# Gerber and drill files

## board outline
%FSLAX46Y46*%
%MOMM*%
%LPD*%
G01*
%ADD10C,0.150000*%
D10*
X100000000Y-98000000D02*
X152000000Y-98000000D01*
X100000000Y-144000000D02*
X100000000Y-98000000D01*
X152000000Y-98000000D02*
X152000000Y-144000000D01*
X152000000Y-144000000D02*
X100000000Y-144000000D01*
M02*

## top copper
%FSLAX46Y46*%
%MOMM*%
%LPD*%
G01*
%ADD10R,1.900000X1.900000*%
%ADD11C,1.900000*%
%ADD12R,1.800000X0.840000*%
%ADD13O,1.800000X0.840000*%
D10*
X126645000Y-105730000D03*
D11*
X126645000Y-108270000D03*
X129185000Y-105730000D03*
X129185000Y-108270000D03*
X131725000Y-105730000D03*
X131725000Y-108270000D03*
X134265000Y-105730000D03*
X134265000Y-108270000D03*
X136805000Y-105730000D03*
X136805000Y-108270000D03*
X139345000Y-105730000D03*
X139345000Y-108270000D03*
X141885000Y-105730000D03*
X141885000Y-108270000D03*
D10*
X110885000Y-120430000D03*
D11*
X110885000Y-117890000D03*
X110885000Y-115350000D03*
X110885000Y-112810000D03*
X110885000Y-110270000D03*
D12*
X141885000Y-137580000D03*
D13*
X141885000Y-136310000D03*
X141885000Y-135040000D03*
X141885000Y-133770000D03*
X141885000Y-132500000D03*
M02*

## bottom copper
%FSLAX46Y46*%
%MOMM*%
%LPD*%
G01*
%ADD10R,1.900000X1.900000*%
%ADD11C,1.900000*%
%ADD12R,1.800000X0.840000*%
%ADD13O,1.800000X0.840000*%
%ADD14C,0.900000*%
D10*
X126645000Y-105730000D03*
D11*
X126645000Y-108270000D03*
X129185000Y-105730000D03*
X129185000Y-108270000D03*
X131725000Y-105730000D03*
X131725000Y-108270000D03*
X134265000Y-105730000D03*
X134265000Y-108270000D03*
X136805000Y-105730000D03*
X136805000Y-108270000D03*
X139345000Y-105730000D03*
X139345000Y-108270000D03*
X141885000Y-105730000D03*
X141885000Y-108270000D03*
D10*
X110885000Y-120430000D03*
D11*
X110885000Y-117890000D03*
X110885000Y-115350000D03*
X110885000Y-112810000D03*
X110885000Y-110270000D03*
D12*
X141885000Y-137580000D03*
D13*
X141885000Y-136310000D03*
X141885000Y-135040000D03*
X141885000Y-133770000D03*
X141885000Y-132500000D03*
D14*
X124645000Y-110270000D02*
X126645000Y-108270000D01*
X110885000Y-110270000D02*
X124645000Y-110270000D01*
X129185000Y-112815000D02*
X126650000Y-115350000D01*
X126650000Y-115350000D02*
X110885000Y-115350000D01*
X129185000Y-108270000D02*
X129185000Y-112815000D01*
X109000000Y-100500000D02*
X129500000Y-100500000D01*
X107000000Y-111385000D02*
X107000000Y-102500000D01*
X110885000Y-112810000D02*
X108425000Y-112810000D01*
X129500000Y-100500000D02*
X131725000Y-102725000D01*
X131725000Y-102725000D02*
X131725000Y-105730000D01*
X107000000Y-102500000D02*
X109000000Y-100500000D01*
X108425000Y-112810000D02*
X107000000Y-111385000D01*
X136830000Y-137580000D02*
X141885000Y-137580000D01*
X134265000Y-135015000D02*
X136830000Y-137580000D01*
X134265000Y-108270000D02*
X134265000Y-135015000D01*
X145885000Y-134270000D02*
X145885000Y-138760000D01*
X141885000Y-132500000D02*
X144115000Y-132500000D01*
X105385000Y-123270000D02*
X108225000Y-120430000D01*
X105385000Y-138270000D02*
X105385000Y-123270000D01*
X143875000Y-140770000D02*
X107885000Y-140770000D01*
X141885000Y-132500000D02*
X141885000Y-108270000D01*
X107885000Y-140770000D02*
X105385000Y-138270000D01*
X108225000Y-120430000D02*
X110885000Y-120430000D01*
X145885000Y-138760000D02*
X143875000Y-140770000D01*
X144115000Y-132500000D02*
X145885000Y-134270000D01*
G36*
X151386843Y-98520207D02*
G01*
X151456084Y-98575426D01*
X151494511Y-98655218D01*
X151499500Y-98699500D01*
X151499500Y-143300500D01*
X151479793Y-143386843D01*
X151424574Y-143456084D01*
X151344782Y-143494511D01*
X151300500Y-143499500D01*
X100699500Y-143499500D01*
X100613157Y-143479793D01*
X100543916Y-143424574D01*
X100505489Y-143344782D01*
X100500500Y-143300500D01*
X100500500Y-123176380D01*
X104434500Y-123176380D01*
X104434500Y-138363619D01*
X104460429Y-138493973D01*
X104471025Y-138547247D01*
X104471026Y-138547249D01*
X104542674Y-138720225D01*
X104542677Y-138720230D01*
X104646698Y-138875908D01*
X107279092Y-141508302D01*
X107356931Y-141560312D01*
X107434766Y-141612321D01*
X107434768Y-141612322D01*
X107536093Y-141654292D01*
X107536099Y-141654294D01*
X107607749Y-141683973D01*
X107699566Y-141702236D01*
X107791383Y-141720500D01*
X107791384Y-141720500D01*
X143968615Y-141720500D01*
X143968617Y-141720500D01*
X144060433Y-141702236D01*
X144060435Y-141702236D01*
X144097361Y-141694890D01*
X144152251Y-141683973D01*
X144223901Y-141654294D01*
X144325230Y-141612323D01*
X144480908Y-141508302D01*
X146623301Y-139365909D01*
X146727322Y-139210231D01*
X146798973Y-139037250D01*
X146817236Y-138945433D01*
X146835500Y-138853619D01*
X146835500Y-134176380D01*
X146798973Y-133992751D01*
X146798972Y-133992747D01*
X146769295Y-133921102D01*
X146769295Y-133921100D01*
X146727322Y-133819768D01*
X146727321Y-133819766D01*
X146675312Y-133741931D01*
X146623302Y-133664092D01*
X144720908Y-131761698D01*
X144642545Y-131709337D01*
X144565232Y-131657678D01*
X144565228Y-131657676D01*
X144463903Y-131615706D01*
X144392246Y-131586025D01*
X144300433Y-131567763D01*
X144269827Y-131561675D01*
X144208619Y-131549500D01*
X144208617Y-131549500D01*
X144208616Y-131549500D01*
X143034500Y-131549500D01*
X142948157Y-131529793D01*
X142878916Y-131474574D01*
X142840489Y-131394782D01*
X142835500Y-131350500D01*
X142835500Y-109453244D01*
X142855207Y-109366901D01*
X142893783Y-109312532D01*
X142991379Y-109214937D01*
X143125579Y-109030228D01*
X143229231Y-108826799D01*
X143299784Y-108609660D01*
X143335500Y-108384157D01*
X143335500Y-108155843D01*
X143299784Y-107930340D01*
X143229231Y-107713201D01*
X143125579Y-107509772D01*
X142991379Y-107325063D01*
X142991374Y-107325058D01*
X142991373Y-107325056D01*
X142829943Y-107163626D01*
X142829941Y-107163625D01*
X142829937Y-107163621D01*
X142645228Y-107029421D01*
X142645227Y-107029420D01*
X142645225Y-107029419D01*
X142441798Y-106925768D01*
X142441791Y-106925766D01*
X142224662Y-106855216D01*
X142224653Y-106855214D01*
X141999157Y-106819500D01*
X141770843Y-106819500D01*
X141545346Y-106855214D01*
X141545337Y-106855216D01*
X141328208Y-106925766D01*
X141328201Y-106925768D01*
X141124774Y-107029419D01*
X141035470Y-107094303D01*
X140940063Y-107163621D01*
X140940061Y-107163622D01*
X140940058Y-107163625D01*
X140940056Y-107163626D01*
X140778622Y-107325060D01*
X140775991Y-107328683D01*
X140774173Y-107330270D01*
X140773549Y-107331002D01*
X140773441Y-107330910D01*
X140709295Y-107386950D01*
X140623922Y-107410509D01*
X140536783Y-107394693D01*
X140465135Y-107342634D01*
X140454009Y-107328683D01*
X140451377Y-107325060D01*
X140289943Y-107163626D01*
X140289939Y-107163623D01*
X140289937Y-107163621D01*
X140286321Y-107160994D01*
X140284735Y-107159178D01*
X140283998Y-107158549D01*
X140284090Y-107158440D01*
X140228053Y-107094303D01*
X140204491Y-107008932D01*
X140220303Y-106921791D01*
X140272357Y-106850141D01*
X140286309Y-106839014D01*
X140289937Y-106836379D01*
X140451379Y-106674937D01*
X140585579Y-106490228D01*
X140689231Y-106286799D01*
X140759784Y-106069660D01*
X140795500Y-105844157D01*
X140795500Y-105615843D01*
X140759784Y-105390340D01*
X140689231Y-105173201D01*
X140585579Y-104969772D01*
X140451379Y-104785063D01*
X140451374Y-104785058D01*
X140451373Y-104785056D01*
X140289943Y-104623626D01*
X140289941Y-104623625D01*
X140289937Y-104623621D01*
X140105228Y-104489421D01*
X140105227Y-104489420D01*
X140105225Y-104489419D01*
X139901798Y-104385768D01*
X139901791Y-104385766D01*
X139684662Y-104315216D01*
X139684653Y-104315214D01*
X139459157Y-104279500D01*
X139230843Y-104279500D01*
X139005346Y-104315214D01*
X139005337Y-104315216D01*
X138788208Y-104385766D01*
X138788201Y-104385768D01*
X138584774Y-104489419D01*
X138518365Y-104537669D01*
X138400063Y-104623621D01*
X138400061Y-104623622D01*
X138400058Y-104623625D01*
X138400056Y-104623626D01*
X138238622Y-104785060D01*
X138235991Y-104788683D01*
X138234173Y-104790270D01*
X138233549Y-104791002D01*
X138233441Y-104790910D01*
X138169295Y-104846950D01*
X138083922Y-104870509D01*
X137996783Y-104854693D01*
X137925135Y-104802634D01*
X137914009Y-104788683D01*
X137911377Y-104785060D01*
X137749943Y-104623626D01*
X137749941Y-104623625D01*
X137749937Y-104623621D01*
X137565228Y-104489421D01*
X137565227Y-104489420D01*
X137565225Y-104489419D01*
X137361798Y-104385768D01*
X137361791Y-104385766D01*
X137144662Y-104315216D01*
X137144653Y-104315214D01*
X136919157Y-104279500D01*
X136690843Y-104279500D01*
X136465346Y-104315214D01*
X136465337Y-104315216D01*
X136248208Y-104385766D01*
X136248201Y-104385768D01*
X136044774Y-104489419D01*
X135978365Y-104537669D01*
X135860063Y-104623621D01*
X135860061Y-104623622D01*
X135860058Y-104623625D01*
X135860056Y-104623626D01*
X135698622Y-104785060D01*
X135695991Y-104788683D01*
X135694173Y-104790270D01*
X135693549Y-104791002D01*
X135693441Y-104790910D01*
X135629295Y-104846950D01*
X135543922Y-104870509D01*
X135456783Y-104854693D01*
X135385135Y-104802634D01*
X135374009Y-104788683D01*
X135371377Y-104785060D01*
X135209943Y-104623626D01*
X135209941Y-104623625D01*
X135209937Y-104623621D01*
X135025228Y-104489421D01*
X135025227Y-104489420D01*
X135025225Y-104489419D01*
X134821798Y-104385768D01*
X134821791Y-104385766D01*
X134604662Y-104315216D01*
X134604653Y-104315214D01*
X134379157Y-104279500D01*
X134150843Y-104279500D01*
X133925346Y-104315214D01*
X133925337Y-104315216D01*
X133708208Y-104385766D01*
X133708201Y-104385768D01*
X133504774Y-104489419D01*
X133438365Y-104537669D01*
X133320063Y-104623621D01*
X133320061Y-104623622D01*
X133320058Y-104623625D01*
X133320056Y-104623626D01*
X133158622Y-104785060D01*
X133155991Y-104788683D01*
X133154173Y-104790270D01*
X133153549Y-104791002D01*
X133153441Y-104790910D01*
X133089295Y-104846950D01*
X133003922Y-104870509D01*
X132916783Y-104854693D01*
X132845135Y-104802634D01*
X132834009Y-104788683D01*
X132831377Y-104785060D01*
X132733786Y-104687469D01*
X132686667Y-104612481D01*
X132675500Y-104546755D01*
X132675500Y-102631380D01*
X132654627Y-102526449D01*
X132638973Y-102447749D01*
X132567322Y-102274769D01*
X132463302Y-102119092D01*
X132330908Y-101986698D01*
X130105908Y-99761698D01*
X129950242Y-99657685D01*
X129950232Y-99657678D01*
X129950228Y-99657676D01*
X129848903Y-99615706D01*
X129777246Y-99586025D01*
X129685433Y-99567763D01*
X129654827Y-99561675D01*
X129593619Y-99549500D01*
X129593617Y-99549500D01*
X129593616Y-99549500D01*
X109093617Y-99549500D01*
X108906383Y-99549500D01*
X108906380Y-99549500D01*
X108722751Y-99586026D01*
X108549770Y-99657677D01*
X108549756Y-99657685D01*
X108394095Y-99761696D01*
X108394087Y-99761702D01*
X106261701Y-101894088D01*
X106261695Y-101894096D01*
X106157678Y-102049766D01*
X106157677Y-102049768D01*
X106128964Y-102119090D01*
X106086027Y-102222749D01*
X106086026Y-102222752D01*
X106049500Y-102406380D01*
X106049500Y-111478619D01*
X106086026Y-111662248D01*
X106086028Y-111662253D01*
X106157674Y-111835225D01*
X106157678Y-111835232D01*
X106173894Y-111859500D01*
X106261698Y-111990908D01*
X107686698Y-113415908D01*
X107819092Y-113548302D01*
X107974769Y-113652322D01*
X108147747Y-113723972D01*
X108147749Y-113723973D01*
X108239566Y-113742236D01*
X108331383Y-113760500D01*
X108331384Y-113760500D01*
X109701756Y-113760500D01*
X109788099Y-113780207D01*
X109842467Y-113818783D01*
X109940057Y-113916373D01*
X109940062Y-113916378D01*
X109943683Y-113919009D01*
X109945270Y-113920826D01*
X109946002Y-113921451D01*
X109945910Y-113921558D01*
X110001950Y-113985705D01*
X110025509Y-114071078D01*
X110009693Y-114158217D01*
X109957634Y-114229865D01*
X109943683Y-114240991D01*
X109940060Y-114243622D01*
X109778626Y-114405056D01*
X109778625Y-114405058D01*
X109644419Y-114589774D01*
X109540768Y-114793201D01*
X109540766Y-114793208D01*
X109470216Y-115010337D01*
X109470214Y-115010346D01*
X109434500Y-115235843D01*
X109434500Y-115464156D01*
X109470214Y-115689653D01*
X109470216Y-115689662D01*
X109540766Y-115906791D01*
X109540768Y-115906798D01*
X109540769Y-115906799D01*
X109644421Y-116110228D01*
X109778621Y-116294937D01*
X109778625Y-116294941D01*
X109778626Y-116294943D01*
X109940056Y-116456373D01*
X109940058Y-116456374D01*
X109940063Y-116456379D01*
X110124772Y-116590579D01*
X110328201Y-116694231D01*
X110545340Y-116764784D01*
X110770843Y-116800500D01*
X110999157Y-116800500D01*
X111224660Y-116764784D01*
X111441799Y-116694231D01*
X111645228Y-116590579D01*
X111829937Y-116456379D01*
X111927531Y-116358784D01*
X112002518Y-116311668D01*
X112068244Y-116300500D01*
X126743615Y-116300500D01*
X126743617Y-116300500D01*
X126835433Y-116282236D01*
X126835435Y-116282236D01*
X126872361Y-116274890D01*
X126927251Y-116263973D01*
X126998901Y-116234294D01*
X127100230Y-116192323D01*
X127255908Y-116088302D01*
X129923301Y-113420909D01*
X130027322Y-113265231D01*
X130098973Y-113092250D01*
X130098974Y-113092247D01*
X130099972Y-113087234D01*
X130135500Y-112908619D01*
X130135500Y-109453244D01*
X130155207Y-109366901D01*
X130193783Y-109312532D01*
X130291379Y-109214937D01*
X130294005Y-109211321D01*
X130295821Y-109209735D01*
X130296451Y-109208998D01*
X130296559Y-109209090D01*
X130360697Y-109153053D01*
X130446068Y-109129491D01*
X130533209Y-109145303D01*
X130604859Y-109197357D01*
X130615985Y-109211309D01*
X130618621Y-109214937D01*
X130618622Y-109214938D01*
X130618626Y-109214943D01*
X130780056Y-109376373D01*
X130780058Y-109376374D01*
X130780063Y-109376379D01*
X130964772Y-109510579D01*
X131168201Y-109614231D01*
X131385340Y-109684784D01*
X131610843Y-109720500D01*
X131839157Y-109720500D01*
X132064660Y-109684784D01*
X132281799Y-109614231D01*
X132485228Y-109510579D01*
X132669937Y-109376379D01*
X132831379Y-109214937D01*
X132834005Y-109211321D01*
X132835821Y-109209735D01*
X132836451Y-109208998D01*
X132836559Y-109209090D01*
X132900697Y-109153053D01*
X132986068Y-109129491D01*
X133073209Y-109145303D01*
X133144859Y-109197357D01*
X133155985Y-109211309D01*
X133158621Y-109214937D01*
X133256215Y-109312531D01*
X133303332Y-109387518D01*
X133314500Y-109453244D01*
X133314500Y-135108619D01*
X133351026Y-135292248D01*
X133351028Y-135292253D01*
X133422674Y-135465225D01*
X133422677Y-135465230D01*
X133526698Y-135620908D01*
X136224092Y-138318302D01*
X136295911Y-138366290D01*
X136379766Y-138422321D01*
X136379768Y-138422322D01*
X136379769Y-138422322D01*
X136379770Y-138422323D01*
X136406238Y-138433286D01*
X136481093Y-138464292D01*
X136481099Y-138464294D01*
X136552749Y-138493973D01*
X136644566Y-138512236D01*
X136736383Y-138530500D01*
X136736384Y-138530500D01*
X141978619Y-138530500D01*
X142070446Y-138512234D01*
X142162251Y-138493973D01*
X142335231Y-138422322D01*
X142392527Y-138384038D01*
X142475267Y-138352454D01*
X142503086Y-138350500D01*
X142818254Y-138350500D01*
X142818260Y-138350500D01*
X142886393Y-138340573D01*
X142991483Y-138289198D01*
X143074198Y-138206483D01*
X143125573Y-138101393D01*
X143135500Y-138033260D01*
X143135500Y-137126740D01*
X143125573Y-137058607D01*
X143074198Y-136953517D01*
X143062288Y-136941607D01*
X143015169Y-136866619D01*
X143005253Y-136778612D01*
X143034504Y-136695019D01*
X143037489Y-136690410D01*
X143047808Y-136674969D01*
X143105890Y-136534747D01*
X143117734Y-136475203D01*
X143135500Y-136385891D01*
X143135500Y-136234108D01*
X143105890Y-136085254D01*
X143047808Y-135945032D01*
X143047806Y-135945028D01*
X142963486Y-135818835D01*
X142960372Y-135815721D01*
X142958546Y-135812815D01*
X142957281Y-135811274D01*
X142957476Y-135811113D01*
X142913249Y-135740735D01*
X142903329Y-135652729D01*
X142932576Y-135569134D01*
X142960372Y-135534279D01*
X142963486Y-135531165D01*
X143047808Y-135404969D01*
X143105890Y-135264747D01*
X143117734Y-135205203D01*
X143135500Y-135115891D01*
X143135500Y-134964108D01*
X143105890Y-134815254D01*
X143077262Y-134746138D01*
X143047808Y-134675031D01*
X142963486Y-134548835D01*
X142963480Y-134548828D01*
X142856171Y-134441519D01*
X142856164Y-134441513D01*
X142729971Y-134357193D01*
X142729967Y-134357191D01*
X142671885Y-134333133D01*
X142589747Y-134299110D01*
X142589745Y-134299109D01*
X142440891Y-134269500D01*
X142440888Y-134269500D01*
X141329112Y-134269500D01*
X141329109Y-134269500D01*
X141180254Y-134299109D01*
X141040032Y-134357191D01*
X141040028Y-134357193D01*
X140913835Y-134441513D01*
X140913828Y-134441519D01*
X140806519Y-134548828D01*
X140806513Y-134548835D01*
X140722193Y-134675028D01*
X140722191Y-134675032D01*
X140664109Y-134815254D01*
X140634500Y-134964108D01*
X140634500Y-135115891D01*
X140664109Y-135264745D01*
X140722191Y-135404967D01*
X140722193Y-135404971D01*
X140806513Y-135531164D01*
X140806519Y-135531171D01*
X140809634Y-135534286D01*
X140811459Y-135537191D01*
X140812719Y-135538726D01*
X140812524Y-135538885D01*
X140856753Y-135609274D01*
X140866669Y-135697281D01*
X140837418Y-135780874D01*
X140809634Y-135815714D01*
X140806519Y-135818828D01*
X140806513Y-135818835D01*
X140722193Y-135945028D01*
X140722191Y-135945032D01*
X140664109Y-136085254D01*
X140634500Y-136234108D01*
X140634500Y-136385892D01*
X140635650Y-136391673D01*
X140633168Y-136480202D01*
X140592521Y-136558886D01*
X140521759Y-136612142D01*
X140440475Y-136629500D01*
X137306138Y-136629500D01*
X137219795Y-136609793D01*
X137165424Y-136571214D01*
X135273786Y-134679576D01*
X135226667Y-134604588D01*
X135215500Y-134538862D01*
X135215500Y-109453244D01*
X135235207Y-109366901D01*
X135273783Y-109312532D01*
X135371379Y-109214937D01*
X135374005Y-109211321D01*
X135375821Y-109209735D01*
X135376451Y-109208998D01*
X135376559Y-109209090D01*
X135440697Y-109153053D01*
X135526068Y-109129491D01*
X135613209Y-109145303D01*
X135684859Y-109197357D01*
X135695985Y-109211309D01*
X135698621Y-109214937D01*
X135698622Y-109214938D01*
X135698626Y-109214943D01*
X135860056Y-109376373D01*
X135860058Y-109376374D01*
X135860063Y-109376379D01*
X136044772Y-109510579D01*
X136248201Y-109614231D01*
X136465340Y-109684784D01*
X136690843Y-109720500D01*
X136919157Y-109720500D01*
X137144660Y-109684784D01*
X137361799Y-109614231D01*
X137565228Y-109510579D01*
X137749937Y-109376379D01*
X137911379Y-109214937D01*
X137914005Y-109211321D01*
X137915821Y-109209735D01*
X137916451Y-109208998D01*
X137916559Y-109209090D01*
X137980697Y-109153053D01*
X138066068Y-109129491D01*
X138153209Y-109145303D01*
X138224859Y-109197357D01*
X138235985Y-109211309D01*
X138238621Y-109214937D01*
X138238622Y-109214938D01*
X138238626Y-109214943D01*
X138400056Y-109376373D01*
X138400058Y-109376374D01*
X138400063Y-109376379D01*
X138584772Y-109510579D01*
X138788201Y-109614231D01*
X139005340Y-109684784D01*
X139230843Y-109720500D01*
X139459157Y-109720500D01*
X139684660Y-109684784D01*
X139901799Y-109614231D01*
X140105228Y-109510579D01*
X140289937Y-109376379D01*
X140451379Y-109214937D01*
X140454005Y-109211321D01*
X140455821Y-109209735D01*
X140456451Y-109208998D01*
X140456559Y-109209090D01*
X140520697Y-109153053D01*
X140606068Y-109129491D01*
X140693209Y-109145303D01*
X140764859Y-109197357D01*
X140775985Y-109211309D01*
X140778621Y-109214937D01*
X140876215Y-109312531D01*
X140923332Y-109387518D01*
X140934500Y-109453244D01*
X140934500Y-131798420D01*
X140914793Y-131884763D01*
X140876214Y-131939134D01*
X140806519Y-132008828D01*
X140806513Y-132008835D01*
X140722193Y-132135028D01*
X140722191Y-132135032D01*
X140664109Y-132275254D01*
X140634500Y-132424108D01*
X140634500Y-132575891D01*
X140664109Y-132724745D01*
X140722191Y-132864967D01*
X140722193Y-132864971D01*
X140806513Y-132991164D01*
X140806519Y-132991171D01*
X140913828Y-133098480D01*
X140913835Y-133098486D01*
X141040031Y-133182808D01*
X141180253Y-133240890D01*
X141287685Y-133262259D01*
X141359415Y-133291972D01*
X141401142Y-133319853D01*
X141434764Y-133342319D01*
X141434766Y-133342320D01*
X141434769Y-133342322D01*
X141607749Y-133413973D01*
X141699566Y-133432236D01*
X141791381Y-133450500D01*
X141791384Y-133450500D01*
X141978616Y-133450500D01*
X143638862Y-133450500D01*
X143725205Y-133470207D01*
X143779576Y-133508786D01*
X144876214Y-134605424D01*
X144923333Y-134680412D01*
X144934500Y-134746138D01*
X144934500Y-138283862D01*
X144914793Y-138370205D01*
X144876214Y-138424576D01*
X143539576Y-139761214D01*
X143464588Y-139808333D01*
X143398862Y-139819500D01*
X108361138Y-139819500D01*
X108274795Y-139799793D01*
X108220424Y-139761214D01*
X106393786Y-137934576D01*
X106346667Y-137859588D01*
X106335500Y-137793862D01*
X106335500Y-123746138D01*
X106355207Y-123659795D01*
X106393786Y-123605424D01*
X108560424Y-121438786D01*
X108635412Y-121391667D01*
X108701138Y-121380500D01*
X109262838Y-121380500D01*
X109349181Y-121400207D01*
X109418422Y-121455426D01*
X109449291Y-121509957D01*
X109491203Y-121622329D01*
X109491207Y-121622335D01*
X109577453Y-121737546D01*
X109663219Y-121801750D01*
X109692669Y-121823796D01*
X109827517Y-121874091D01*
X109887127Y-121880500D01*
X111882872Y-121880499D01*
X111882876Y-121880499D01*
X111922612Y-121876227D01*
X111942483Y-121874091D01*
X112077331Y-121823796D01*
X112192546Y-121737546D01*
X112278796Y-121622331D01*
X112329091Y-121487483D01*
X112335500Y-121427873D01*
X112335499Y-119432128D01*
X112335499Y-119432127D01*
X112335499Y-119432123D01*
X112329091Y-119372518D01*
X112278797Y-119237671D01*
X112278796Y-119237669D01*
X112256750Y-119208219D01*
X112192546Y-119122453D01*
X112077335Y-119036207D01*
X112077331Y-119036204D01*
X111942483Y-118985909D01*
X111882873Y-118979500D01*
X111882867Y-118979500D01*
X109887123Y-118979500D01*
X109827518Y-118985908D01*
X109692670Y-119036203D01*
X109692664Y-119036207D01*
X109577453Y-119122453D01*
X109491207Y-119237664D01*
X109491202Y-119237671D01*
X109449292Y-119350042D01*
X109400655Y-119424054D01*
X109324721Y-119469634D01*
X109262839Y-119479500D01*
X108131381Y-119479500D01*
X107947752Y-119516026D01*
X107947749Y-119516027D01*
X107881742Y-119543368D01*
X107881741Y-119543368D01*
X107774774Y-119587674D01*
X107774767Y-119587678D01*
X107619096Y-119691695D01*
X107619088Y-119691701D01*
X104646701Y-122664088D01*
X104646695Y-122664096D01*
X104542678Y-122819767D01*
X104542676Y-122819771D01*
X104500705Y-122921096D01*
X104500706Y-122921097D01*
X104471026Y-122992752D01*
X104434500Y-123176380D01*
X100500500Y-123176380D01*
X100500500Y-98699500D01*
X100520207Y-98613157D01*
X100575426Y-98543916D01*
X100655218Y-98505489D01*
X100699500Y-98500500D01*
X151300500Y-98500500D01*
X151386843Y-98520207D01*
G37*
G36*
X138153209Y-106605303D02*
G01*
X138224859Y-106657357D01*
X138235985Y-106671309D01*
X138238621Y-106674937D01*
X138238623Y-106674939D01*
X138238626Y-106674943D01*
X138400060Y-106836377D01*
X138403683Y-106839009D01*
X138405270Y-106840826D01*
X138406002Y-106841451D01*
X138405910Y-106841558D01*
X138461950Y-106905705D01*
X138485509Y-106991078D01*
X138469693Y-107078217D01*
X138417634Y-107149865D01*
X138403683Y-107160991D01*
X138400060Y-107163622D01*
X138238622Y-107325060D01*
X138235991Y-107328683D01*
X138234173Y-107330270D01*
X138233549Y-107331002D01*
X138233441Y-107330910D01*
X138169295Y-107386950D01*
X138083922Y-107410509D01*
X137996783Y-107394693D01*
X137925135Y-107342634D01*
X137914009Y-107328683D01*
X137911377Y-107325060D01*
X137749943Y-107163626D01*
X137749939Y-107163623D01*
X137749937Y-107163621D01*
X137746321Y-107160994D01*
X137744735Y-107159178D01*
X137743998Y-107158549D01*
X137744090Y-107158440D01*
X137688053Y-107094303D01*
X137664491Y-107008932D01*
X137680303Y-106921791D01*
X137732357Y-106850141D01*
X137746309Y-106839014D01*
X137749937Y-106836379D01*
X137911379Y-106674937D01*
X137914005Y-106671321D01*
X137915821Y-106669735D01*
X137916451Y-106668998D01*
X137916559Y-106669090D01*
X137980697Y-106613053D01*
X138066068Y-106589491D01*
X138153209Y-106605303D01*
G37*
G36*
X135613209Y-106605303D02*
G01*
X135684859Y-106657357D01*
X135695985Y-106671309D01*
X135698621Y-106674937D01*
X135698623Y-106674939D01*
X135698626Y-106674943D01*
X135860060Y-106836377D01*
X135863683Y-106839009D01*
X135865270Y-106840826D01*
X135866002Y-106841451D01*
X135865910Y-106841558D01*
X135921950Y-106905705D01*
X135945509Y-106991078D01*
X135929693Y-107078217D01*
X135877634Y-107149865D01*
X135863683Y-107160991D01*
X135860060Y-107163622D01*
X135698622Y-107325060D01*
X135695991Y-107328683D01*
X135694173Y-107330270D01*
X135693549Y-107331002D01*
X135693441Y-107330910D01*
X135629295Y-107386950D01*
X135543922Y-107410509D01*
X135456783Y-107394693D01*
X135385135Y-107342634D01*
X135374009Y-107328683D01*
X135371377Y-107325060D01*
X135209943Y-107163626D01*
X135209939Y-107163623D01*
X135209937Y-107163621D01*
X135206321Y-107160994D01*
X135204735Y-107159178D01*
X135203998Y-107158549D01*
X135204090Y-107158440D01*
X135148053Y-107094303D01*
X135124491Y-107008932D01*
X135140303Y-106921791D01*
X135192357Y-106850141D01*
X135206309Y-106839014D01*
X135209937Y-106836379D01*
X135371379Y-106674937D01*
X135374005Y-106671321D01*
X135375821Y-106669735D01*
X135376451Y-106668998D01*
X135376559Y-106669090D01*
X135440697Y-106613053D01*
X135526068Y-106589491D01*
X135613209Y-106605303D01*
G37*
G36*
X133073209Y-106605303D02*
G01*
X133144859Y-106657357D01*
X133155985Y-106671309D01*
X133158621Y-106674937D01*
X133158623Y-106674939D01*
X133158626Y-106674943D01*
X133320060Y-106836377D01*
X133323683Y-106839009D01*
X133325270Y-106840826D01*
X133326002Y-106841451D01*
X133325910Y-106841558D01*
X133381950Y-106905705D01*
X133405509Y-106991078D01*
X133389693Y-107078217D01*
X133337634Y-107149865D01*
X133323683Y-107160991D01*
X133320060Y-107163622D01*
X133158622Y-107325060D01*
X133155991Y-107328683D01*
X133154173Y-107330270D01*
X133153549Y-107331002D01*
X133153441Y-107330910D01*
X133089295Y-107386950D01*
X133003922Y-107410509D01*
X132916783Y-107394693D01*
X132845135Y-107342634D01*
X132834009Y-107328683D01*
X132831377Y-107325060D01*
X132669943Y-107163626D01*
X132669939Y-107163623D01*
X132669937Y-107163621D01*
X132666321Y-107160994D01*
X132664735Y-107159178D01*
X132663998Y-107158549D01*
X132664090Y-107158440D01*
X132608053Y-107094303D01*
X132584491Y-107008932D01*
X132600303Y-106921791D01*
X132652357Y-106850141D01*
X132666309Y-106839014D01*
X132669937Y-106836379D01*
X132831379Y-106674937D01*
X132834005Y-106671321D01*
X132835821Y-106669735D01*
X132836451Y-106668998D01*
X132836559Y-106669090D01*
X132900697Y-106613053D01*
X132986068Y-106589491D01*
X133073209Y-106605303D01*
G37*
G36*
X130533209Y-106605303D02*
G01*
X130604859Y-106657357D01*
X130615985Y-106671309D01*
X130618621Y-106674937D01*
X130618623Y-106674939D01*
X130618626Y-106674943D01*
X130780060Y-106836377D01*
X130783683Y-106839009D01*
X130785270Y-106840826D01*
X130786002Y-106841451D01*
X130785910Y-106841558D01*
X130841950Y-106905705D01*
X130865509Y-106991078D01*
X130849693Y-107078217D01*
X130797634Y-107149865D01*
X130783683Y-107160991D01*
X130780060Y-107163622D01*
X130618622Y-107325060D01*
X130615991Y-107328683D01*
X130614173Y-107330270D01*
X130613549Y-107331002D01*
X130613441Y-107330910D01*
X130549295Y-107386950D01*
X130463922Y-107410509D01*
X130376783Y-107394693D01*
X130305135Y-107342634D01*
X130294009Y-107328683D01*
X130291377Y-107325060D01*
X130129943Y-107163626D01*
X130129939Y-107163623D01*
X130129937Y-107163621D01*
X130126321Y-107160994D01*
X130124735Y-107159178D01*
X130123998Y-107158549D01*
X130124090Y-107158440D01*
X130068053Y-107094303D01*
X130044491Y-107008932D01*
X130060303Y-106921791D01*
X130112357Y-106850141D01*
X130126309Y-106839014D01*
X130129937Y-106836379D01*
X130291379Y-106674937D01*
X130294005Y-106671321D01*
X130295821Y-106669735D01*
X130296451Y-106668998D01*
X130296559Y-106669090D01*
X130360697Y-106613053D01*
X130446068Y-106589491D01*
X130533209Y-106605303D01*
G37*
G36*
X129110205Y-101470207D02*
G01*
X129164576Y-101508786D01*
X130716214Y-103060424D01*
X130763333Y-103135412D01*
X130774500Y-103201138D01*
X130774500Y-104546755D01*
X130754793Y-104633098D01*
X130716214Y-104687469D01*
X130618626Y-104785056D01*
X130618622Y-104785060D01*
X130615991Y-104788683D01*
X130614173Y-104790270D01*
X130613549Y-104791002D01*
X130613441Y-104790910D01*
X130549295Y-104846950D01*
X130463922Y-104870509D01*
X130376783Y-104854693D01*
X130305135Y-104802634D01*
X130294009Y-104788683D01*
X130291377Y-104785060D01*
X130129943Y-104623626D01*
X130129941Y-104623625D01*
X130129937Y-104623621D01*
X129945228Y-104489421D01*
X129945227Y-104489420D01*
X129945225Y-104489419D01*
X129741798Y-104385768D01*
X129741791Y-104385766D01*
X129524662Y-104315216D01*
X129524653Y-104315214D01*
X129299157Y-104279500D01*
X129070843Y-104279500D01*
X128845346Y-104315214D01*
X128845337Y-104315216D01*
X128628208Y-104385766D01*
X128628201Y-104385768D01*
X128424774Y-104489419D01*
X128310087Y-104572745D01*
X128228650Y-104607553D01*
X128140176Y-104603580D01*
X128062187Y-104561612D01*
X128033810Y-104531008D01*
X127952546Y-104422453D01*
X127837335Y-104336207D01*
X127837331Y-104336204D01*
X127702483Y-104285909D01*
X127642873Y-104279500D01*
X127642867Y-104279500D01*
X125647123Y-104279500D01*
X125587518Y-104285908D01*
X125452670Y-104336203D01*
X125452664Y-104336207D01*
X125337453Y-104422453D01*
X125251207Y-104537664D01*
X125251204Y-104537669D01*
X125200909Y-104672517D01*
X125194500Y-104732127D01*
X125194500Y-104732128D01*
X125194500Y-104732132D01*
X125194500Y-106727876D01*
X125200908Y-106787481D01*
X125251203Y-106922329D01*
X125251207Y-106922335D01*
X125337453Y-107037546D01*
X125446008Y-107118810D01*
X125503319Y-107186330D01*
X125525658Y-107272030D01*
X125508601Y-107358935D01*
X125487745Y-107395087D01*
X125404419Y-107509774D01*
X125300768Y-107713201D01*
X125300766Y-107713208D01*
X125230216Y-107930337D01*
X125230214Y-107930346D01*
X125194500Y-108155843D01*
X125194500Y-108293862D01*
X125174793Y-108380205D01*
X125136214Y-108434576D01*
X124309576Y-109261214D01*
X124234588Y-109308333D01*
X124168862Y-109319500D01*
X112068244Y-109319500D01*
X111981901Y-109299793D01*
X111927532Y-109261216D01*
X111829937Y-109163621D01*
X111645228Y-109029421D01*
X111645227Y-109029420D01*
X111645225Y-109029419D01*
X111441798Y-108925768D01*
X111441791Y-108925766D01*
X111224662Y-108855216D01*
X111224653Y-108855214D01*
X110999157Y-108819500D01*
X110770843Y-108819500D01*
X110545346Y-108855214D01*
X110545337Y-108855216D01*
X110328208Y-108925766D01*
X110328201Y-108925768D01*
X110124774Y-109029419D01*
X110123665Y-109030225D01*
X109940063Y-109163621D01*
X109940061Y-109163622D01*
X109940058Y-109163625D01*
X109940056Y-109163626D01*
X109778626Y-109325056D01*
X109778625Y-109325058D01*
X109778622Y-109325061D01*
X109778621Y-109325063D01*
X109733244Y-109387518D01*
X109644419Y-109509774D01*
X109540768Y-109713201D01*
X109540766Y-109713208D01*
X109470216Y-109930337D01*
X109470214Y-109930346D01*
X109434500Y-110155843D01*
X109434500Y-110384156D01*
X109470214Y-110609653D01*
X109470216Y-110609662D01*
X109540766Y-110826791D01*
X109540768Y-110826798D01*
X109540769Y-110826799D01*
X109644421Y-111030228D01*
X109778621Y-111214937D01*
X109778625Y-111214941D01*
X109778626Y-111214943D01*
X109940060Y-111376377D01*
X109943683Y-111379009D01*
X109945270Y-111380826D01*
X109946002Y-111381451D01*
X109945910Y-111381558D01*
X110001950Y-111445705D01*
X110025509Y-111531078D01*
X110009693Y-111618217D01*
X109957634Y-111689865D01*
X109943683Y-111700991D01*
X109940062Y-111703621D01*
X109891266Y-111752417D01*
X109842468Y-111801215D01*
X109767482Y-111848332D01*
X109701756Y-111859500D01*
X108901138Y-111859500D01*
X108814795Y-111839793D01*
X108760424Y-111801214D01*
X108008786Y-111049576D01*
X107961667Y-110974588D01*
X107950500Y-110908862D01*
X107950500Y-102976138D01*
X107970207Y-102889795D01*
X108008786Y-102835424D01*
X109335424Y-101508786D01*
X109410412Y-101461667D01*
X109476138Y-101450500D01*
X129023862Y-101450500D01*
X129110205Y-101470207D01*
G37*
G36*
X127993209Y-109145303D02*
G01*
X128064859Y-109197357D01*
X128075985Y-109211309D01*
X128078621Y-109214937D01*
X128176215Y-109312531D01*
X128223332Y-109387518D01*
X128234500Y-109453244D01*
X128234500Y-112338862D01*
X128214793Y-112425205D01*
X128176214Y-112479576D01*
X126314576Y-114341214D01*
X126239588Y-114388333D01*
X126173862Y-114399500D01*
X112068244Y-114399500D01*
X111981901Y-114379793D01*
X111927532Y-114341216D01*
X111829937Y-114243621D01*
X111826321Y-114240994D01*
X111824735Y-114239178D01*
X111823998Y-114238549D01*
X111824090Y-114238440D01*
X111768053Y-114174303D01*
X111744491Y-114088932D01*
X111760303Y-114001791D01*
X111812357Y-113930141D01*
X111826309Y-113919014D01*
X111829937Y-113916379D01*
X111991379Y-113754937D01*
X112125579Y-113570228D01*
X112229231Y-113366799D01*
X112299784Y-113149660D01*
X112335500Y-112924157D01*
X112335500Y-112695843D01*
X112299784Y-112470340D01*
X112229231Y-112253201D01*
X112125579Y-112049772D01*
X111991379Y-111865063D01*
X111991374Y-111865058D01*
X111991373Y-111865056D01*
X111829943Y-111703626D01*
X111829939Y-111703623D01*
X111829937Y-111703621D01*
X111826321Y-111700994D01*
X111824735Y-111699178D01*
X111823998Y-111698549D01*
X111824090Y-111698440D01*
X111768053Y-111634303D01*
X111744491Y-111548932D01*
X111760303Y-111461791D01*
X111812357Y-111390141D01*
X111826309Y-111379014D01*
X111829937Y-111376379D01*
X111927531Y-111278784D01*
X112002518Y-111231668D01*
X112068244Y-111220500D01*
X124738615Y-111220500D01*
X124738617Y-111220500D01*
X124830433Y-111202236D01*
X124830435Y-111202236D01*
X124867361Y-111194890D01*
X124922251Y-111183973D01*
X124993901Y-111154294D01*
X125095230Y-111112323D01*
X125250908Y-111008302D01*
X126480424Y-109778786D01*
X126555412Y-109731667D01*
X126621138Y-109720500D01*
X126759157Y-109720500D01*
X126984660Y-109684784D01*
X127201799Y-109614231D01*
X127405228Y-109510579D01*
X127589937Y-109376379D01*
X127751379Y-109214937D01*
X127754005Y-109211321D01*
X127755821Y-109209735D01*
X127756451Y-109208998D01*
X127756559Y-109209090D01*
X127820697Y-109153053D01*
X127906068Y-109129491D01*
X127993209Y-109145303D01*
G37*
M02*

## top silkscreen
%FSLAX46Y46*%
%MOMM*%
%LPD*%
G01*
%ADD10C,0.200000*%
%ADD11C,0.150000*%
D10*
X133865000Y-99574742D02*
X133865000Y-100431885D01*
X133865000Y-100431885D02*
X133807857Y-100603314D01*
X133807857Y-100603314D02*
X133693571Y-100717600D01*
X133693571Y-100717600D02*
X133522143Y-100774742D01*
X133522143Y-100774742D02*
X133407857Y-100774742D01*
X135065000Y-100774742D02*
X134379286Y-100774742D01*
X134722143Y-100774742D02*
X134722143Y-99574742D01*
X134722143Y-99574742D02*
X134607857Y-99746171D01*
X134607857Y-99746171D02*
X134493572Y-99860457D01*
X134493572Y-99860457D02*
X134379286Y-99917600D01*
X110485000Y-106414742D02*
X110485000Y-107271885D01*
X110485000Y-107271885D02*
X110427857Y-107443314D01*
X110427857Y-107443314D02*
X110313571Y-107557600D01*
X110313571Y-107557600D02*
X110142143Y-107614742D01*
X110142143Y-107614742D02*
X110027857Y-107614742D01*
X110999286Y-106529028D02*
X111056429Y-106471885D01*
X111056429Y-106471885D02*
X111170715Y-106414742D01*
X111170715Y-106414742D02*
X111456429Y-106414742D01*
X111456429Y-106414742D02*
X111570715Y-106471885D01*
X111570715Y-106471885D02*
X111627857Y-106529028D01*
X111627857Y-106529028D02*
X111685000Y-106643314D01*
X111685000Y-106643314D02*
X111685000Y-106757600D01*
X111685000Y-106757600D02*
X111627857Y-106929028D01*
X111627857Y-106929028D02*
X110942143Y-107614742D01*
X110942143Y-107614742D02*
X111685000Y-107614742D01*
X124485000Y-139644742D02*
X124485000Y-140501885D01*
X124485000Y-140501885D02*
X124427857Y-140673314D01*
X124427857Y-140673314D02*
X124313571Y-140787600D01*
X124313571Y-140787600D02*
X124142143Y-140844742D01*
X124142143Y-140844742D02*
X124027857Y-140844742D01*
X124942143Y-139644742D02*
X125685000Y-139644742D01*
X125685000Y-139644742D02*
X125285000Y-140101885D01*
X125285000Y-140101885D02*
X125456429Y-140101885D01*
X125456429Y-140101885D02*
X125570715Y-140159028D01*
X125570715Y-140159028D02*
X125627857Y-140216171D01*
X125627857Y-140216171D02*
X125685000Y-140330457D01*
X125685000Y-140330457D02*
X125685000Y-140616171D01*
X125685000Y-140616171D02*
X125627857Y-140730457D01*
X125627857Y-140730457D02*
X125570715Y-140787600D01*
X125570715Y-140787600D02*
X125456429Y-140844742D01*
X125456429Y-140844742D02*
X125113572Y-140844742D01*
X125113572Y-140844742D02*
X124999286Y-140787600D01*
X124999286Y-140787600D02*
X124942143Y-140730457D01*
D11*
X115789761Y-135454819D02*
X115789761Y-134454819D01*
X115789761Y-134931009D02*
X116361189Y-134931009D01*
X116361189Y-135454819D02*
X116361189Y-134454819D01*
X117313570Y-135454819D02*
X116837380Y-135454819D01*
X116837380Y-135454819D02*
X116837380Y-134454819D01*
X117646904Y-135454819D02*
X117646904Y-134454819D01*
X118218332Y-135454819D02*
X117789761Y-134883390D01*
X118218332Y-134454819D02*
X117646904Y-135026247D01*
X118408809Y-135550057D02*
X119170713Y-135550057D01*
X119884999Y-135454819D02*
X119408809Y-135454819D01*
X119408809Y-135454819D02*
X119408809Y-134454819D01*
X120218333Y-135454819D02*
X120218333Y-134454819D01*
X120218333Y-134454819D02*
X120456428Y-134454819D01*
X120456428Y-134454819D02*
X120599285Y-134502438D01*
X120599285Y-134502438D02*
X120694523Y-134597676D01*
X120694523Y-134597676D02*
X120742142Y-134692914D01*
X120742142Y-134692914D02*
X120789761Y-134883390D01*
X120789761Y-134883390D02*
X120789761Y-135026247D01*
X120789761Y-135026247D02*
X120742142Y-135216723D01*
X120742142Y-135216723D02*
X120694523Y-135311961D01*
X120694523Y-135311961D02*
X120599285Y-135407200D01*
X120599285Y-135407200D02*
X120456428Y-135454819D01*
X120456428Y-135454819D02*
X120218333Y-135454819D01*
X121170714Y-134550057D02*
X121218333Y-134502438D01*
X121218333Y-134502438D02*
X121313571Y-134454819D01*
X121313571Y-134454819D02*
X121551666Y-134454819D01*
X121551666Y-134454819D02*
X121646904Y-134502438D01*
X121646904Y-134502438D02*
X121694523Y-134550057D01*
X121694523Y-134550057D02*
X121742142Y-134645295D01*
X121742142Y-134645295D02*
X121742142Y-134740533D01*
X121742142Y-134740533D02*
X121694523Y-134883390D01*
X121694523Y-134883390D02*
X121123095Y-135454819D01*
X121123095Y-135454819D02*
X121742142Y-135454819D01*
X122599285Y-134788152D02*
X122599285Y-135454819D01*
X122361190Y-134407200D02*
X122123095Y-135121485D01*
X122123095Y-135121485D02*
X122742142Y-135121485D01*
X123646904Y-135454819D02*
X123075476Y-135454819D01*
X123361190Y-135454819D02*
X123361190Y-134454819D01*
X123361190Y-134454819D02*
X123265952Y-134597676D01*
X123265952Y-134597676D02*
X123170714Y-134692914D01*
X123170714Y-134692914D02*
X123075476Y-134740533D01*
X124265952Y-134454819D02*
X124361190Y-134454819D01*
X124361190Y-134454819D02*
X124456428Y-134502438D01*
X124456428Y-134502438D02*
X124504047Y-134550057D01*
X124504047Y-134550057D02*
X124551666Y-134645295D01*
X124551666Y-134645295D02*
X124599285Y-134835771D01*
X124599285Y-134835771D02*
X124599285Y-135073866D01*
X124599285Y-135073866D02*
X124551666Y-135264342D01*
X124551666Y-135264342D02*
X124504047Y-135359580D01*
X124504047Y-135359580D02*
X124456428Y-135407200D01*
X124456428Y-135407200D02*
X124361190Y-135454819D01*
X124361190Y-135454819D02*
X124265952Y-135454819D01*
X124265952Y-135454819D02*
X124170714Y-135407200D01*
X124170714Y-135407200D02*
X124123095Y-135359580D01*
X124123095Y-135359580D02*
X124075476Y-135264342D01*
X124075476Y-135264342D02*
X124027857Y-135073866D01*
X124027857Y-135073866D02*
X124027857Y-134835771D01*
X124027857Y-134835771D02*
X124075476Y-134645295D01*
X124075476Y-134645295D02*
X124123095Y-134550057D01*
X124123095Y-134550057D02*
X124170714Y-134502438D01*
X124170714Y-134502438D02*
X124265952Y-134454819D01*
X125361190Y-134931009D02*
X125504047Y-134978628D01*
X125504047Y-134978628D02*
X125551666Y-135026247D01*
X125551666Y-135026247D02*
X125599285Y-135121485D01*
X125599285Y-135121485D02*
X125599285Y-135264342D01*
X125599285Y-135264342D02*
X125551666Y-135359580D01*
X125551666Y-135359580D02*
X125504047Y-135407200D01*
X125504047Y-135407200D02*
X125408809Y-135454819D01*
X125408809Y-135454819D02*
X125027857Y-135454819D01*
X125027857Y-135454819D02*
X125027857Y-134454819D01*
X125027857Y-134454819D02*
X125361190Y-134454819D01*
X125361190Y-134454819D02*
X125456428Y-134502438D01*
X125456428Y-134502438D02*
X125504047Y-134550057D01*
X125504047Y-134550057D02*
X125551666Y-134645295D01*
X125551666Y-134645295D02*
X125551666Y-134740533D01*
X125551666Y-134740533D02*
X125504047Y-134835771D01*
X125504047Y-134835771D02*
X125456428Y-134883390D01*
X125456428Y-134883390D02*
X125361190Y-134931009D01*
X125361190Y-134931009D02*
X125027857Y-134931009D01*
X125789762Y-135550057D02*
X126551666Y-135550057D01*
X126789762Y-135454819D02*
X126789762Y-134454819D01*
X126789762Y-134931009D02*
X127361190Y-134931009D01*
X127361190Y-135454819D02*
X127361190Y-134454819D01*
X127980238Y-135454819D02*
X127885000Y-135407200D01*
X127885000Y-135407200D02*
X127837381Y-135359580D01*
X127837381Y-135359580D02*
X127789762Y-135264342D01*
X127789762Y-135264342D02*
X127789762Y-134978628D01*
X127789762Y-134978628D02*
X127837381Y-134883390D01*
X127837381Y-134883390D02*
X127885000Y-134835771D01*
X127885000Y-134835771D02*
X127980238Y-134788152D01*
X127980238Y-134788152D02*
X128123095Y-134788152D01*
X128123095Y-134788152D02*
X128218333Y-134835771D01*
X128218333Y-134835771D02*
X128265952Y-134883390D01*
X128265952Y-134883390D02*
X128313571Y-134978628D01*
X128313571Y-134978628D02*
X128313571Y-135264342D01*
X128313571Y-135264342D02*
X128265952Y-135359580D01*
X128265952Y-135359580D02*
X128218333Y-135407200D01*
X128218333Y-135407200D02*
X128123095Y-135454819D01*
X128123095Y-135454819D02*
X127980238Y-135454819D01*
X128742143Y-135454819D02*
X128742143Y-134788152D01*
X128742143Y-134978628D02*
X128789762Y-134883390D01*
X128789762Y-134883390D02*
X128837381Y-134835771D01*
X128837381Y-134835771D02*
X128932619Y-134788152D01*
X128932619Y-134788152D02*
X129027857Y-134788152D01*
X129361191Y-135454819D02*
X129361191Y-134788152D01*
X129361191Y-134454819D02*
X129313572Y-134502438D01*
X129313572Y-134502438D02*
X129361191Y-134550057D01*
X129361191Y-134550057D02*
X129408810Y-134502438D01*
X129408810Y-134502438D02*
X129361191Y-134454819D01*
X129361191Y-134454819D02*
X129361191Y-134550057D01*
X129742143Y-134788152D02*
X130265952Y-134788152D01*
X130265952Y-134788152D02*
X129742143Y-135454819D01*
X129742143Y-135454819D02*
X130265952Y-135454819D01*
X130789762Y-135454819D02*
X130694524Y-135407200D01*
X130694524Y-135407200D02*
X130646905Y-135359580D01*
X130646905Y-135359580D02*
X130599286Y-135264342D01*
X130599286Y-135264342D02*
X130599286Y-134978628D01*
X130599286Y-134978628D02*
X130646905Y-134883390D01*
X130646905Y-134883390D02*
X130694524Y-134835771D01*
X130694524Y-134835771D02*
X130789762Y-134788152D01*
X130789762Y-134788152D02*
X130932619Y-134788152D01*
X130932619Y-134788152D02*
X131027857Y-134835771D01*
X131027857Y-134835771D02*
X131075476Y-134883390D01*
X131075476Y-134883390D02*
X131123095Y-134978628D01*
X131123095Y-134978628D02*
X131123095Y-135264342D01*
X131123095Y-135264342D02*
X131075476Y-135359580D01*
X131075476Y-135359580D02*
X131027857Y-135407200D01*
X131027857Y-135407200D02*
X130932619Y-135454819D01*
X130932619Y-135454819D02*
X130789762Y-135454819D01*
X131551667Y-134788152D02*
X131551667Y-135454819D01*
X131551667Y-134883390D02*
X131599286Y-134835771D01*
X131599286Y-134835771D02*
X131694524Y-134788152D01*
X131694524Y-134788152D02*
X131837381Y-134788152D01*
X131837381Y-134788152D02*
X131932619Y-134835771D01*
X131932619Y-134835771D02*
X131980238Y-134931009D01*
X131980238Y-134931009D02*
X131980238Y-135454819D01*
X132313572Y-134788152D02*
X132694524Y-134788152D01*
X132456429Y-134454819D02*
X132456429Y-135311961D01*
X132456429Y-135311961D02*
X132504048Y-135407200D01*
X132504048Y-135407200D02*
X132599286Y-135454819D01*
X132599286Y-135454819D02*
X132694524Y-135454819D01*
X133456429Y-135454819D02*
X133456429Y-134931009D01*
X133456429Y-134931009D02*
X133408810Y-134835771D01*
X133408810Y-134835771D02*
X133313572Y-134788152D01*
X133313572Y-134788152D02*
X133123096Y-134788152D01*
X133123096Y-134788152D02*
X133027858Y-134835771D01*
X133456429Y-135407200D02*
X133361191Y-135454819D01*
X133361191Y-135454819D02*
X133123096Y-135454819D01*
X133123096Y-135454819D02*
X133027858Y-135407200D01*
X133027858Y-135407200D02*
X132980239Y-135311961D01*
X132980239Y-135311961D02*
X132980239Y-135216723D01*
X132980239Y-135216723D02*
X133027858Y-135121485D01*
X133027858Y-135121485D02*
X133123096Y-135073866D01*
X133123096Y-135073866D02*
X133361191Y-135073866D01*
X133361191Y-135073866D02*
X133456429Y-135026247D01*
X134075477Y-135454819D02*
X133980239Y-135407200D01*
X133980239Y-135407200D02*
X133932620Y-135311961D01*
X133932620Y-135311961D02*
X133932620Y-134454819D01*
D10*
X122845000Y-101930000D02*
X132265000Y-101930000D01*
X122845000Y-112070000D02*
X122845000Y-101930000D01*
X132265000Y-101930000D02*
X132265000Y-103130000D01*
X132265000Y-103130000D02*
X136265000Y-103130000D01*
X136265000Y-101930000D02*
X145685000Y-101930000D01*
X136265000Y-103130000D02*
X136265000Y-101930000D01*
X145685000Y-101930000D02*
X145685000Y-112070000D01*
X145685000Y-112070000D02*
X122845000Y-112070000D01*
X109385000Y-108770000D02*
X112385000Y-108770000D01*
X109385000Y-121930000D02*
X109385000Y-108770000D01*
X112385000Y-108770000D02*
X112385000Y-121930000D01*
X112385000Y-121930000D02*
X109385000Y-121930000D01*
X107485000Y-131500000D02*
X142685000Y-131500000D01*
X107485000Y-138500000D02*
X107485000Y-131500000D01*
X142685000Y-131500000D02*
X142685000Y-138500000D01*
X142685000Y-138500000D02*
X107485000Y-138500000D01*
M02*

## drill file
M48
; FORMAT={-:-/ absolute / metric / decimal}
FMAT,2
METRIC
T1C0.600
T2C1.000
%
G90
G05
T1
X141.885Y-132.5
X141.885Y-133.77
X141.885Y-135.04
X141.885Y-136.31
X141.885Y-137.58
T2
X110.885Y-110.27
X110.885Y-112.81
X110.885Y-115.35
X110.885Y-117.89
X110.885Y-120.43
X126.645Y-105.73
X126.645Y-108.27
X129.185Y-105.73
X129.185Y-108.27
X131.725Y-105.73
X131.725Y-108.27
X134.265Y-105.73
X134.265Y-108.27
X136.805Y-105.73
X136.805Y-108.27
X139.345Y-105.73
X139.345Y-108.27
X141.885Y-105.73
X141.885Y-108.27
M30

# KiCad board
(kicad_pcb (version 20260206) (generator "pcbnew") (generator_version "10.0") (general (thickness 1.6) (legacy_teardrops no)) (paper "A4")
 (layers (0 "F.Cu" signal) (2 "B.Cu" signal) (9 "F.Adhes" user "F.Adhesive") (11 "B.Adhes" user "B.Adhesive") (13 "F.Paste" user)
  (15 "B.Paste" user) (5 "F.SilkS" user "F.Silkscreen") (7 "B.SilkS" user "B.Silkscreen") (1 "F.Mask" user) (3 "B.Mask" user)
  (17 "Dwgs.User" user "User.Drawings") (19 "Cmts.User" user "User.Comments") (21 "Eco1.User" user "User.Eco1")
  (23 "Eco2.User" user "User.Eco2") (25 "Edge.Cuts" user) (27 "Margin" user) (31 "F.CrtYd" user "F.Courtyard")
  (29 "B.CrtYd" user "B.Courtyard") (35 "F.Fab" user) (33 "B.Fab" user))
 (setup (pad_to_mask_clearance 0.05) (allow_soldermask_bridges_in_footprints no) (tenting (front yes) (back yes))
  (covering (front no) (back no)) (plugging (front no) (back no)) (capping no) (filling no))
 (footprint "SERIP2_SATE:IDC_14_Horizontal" (layer "F.Cu") (at 126.645 105.73)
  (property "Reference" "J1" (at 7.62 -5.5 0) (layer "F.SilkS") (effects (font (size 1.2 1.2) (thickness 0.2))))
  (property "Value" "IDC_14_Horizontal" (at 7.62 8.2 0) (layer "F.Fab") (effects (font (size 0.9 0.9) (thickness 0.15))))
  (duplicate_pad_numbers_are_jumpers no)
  (fp_line (start -3.8 -3.8) (end 5.62 -3.8) (stroke (width 0.2) (type solid)) (layer "F.SilkS"))
  (fp_line (start -3.8 6.34) (end -3.8 -3.8) (stroke (width 0.2) (type solid)) (layer "F.SilkS"))
  (fp_line (start 5.62 -3.8) (end 5.62 -2.6) (stroke (width 0.2) (type solid)) (layer "F.SilkS"))
  (fp_line (start 5.62 -2.6) (end 9.62 -2.6) (stroke (width 0.2) (type solid)) (layer "F.SilkS"))
  (fp_line (start 9.62 -3.8) (end 19.04 -3.8) (stroke (width 0.2) (type solid)) (layer "F.SilkS"))
  (fp_line (start 9.62 -2.6) (end 9.62 -3.8) (stroke (width 0.2) (type solid)) (layer "F.SilkS"))
  (fp_line (start 19.04 -3.8) (end 19.04 6.34) (stroke (width 0.2) (type solid)) (layer "F.SilkS"))
  (fp_line (start 19.04 6.34) (end -3.8 6.34) (stroke (width 0.2) (type solid)) (layer "F.SilkS"))
  (pad "1" thru_hole rect (at 0 0) (size 1.9 1.9) (drill 1) (layers "*.Cu" "B.Mask") (remove_unused_layers no)
   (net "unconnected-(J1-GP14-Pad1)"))
  (pad "2" thru_hole circle (at 0 2.54) (size 1.9 1.9) (drill 1) (layers "*.Cu" "B.Mask") (remove_unused_layers no) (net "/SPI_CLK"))
  (pad "3" thru_hole circle (at 2.54 0) (size 1.9 1.9) (drill 1) (layers "*.Cu" "B.Mask") (remove_unused_layers no)
   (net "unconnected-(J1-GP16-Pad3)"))
  (pad "4" thru_hole circle (at 2.54 2.54) (size 1.9 1.9) (drill 1) (layers "*.Cu" "B.Mask") (remove_unused_layers no) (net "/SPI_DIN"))
  (pad "5" thru_hole circle (at 5.08 0) (size 1.9 1.9) (drill 1) (layers "*.Cu" "B.Mask") (remove_unused_layers no) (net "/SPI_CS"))
  (pad "6" thru_hole circle (at 5.08 2.54) (size 1.9 1.9) (drill 1) (layers "*.Cu" "B.Mask") (remove_unused_layers no)
   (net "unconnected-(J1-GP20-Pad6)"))
  (pad "7" thru_hole circle (at 7.62 0) (size 1.9 1.9) (drill 1) (layers "*.Cu" "B.Mask") (remove_unused_layers no)
   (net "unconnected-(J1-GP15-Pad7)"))
  (pad "8" thru_hole circle (at 7.62 2.54) (size 1.9 1.9) (drill 1) (layers "*.Cu" "B.Mask") (remove_unused_layers no) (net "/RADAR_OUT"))
  (pad "9" thru_hole circle (at 10.16 0) (size 1.9 1.9) (drill 1) (layers "*.Cu" "B.Mask") (remove_unused_layers no)
   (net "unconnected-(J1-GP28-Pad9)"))
  (pad "10" thru_hole circle (at 10.16 2.54) (size 1.9 1.9) (drill 1) (layers "*.Cu" "B.Mask") (remove_unused_layers no)
   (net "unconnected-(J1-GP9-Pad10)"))
  (pad "11" thru_hole circle (at 12.7 0) (size 1.9 1.9) (drill 1) (layers "*.Cu" "B.Mask") (remove_unused_layers no)
   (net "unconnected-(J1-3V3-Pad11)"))
  (pad "12" thru_hole circle (at 12.7 2.54) (size 1.9 1.9) (drill 1) (layers "*.Cu" "B.Mask") (remove_unused_layers no)
   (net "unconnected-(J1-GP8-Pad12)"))
  (pad "13" thru_hole circle (at 15.24 0) (size 1.9 1.9) (drill 1) (layers "*.Cu" "B.Mask") (remove_unused_layers no) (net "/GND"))
  (pad "14" thru_hole circle (at 15.24 2.54) (size 1.9 1.9) (drill 1) (layers "*.Cu" "B.Mask") (remove_unused_layers no) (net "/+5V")))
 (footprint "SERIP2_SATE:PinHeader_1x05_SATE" (layer "F.Cu") (at 110.885 110.27)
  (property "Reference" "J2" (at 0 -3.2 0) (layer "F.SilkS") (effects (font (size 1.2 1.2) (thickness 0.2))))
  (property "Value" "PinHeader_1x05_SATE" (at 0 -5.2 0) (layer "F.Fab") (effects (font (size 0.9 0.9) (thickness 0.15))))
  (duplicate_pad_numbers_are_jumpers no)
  (fp_line (start -1.5 -1.5) (end 1.5 -1.5) (stroke (width 0.2) (type solid)) (layer "F.SilkS"))
  (fp_line (start -1.5 11.66) (end -1.5 -1.5) (stroke (width 0.2) (type solid)) (layer "F.SilkS"))
  (fp_line (start 1.5 -1.5) (end 1.5 11.66) (stroke (width 0.2) (type solid)) (layer "F.SilkS"))
  (fp_line (start 1.5 11.66) (end -1.5 11.66) (stroke (width 0.2) (type solid)) (layer "F.SilkS"))
  (pad "1" thru_hole rect (at 0 10.16) (size 1.9 1.9) (drill 1) (layers "*.Cu" "B.Mask") (remove_unused_layers no) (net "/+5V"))
  (pad "2" thru_hole circle (at 0 7.62) (size 1.9 1.9) (drill 1) (layers "*.Cu" "B.Mask") (remove_unused_layers no) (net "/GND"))
  (pad "3" thru_hole circle (at 0 5.08) (size 1.9 1.9) (drill 1) (layers "*.Cu" "B.Mask") (remove_unused_layers no) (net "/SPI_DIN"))
  (pad "4" thru_hole circle (at 0 2.54) (size 1.9 1.9) (drill 1) (layers "*.Cu" "B.Mask") (remove_unused_layers no) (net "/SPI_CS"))
  (pad "5" thru_hole circle (at 0 0) (size 1.9 1.9) (drill 1) (layers "*.Cu" "B.Mask") (remove_unused_layers no) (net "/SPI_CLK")))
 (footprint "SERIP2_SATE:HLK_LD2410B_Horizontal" (layer "F.Cu") (at 141.885 132.5)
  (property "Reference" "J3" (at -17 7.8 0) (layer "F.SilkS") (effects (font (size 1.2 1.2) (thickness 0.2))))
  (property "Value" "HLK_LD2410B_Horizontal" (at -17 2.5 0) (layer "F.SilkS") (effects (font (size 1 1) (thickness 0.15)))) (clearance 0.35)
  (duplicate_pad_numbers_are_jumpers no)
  (fp_line (start -34.4 -1) (end 0.8 -1) (stroke (width 0.2) (type solid)) (layer "F.SilkS"))
  (fp_line (start -34.4 6) (end -34.4 -1) (stroke (width 0.2) (type solid)) (layer "F.SilkS"))
  (fp_line (start 0.8 -1) (end 0.8 6) (stroke (width 0.2) (type solid)) (layer "F.SilkS"))
  (fp_line (start 0.8 6) (end -34.4 6) (stroke (width 0.2) (type solid)) (layer "F.SilkS"))
  (pad "1" thru_hole rect (at 0 5.08) (size 1.8 0.84) (drill 0.6) (layers "*.Cu" "B.Mask") (remove_unused_layers no) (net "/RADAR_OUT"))
  (pad "2" thru_hole oval (at 0 3.81) (size 1.8 0.84) (drill 0.6) (layers "*.Cu" "B.Mask") (remove_unused_layers no)
   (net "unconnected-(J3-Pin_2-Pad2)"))
  (pad "3" thru_hole oval (at 0 2.54) (size 1.8 0.84) (drill 0.6) (layers "*.Cu" "B.Mask") (remove_unused_layers no)
   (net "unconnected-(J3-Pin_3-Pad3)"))
  (pad "4" thru_hole oval (at 0 1.27) (size 1.8 0.84) (drill 0.6) (layers "*.Cu" "B.Mask") (remove_unused_layers no) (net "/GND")
   (zone_connect 2))
  (pad "5" thru_hole oval (at 0 0) (size 1.8 0.84) (drill 0.6) (layers "*.Cu" "B.Mask") (remove_unused_layers no) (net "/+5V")))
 (gr_line (start 100 98) (end 152 98) (stroke (width 0.15) (type solid)) (layer "Edge.Cuts"))
 (gr_line (start 100 144) (end 100 98) (stroke (width 0.15) (type solid)) (layer "Edge.Cuts"))
 (gr_line (start 152 98) (end 152 144) (stroke (width 0.15) (type solid)) (layer "Edge.Cuts"))
 (gr_line (start 152 144) (end 100 144) (stroke (width 0.15) (type solid)) (layer "Edge.Cuts"))
 (segment (start 124.645 110.27) (end 126.645 108.27) (width 0.9) (layer "B.Cu") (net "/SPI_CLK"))
 (segment (start 110.885 110.27) (end 124.645 110.27) (width 0.9) (layer "B.Cu") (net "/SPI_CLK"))
 (segment (start 129.185 112.815) (end 126.65 115.35) (width 0.9) (layer "B.Cu") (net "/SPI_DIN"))
 (segment (start 126.65 115.35) (end 110.885 115.35) (width 0.9) (layer "B.Cu") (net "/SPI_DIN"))
 (segment (start 129.185 108.27) (end 129.185 112.815) (width 0.9) (layer "B.Cu") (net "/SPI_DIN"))
 (segment (start 109 100.5) (end 129.5 100.5) (width 0.9) (layer "B.Cu") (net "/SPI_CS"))
 (segment (start 107 111.385) (end 107 102.5) (width 0.9) (layer "B.Cu") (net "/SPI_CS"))
 (segment (start 110.885 112.81) (end 108.425 112.81) (width 0.9) (layer "B.Cu") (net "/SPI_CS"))
 (segment (start 129.5 100.5) (end 131.725 102.725) (width 0.9) (layer "B.Cu") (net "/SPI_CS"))
 (segment (start 131.725 102.725) (end 131.725 105.73) (width 0.9) (layer "B.Cu") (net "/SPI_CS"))
 (segment (start 107 102.5) (end 109 100.5) (width 0.9) (layer "B.Cu") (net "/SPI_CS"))
 (segment (start 108.425 112.81) (end 107 111.385) (width 0.9) (layer "B.Cu") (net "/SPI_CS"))
 (segment (start 136.83 137.58) (end 141.885 137.58) (width 0.9) (layer "B.Cu") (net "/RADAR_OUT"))
 (segment (start 134.265 135.015) (end 136.83 137.58) (width 0.9) (layer "B.Cu") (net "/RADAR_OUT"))
 (segment (start 134.265 108.27) (end 134.265 135.015) (width 0.9) (layer "B.Cu") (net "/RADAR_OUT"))
 (segment (start 145.885 134.27) (end 145.885 138.76) (width 0.9) (layer "B.Cu") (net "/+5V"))
 (segment (start 141.885 132.5) (end 144.115 132.5) (width 0.9) (layer "B.Cu") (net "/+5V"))
 (segment (start 105.385 123.27) (end 108.225 120.43) (width 0.9) (layer "B.Cu") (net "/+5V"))
 (segment (start 105.385 138.27) (end 105.385 123.27) (width 0.9) (layer "B.Cu") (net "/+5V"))
 (segment (start 143.875 140.77) (end 107.885 140.77) (width 0.9) (layer "B.Cu") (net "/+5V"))
 (segment (start 141.885 132.5) (end 141.885 108.27) (width 0.9) (layer "B.Cu") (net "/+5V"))
 (segment (start 107.885 140.77) (end 105.385 138.27) (width 0.9) (layer "B.Cu") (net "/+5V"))
 (segment (start 108.225 120.43) (end 110.885 120.43) (width 0.9) (layer "B.Cu") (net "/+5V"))
 (segment (start 145.885 138.76) (end 143.875 140.77) (width 0.9) (layer "B.Cu") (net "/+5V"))
 (segment (start 144.115 132.5) (end 145.885 134.27) (width 0.9) (layer "B.Cu") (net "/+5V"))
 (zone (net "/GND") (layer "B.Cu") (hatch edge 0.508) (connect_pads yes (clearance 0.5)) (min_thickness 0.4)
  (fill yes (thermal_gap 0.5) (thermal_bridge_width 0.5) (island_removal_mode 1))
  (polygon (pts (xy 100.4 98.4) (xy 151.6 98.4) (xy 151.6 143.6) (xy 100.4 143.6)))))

